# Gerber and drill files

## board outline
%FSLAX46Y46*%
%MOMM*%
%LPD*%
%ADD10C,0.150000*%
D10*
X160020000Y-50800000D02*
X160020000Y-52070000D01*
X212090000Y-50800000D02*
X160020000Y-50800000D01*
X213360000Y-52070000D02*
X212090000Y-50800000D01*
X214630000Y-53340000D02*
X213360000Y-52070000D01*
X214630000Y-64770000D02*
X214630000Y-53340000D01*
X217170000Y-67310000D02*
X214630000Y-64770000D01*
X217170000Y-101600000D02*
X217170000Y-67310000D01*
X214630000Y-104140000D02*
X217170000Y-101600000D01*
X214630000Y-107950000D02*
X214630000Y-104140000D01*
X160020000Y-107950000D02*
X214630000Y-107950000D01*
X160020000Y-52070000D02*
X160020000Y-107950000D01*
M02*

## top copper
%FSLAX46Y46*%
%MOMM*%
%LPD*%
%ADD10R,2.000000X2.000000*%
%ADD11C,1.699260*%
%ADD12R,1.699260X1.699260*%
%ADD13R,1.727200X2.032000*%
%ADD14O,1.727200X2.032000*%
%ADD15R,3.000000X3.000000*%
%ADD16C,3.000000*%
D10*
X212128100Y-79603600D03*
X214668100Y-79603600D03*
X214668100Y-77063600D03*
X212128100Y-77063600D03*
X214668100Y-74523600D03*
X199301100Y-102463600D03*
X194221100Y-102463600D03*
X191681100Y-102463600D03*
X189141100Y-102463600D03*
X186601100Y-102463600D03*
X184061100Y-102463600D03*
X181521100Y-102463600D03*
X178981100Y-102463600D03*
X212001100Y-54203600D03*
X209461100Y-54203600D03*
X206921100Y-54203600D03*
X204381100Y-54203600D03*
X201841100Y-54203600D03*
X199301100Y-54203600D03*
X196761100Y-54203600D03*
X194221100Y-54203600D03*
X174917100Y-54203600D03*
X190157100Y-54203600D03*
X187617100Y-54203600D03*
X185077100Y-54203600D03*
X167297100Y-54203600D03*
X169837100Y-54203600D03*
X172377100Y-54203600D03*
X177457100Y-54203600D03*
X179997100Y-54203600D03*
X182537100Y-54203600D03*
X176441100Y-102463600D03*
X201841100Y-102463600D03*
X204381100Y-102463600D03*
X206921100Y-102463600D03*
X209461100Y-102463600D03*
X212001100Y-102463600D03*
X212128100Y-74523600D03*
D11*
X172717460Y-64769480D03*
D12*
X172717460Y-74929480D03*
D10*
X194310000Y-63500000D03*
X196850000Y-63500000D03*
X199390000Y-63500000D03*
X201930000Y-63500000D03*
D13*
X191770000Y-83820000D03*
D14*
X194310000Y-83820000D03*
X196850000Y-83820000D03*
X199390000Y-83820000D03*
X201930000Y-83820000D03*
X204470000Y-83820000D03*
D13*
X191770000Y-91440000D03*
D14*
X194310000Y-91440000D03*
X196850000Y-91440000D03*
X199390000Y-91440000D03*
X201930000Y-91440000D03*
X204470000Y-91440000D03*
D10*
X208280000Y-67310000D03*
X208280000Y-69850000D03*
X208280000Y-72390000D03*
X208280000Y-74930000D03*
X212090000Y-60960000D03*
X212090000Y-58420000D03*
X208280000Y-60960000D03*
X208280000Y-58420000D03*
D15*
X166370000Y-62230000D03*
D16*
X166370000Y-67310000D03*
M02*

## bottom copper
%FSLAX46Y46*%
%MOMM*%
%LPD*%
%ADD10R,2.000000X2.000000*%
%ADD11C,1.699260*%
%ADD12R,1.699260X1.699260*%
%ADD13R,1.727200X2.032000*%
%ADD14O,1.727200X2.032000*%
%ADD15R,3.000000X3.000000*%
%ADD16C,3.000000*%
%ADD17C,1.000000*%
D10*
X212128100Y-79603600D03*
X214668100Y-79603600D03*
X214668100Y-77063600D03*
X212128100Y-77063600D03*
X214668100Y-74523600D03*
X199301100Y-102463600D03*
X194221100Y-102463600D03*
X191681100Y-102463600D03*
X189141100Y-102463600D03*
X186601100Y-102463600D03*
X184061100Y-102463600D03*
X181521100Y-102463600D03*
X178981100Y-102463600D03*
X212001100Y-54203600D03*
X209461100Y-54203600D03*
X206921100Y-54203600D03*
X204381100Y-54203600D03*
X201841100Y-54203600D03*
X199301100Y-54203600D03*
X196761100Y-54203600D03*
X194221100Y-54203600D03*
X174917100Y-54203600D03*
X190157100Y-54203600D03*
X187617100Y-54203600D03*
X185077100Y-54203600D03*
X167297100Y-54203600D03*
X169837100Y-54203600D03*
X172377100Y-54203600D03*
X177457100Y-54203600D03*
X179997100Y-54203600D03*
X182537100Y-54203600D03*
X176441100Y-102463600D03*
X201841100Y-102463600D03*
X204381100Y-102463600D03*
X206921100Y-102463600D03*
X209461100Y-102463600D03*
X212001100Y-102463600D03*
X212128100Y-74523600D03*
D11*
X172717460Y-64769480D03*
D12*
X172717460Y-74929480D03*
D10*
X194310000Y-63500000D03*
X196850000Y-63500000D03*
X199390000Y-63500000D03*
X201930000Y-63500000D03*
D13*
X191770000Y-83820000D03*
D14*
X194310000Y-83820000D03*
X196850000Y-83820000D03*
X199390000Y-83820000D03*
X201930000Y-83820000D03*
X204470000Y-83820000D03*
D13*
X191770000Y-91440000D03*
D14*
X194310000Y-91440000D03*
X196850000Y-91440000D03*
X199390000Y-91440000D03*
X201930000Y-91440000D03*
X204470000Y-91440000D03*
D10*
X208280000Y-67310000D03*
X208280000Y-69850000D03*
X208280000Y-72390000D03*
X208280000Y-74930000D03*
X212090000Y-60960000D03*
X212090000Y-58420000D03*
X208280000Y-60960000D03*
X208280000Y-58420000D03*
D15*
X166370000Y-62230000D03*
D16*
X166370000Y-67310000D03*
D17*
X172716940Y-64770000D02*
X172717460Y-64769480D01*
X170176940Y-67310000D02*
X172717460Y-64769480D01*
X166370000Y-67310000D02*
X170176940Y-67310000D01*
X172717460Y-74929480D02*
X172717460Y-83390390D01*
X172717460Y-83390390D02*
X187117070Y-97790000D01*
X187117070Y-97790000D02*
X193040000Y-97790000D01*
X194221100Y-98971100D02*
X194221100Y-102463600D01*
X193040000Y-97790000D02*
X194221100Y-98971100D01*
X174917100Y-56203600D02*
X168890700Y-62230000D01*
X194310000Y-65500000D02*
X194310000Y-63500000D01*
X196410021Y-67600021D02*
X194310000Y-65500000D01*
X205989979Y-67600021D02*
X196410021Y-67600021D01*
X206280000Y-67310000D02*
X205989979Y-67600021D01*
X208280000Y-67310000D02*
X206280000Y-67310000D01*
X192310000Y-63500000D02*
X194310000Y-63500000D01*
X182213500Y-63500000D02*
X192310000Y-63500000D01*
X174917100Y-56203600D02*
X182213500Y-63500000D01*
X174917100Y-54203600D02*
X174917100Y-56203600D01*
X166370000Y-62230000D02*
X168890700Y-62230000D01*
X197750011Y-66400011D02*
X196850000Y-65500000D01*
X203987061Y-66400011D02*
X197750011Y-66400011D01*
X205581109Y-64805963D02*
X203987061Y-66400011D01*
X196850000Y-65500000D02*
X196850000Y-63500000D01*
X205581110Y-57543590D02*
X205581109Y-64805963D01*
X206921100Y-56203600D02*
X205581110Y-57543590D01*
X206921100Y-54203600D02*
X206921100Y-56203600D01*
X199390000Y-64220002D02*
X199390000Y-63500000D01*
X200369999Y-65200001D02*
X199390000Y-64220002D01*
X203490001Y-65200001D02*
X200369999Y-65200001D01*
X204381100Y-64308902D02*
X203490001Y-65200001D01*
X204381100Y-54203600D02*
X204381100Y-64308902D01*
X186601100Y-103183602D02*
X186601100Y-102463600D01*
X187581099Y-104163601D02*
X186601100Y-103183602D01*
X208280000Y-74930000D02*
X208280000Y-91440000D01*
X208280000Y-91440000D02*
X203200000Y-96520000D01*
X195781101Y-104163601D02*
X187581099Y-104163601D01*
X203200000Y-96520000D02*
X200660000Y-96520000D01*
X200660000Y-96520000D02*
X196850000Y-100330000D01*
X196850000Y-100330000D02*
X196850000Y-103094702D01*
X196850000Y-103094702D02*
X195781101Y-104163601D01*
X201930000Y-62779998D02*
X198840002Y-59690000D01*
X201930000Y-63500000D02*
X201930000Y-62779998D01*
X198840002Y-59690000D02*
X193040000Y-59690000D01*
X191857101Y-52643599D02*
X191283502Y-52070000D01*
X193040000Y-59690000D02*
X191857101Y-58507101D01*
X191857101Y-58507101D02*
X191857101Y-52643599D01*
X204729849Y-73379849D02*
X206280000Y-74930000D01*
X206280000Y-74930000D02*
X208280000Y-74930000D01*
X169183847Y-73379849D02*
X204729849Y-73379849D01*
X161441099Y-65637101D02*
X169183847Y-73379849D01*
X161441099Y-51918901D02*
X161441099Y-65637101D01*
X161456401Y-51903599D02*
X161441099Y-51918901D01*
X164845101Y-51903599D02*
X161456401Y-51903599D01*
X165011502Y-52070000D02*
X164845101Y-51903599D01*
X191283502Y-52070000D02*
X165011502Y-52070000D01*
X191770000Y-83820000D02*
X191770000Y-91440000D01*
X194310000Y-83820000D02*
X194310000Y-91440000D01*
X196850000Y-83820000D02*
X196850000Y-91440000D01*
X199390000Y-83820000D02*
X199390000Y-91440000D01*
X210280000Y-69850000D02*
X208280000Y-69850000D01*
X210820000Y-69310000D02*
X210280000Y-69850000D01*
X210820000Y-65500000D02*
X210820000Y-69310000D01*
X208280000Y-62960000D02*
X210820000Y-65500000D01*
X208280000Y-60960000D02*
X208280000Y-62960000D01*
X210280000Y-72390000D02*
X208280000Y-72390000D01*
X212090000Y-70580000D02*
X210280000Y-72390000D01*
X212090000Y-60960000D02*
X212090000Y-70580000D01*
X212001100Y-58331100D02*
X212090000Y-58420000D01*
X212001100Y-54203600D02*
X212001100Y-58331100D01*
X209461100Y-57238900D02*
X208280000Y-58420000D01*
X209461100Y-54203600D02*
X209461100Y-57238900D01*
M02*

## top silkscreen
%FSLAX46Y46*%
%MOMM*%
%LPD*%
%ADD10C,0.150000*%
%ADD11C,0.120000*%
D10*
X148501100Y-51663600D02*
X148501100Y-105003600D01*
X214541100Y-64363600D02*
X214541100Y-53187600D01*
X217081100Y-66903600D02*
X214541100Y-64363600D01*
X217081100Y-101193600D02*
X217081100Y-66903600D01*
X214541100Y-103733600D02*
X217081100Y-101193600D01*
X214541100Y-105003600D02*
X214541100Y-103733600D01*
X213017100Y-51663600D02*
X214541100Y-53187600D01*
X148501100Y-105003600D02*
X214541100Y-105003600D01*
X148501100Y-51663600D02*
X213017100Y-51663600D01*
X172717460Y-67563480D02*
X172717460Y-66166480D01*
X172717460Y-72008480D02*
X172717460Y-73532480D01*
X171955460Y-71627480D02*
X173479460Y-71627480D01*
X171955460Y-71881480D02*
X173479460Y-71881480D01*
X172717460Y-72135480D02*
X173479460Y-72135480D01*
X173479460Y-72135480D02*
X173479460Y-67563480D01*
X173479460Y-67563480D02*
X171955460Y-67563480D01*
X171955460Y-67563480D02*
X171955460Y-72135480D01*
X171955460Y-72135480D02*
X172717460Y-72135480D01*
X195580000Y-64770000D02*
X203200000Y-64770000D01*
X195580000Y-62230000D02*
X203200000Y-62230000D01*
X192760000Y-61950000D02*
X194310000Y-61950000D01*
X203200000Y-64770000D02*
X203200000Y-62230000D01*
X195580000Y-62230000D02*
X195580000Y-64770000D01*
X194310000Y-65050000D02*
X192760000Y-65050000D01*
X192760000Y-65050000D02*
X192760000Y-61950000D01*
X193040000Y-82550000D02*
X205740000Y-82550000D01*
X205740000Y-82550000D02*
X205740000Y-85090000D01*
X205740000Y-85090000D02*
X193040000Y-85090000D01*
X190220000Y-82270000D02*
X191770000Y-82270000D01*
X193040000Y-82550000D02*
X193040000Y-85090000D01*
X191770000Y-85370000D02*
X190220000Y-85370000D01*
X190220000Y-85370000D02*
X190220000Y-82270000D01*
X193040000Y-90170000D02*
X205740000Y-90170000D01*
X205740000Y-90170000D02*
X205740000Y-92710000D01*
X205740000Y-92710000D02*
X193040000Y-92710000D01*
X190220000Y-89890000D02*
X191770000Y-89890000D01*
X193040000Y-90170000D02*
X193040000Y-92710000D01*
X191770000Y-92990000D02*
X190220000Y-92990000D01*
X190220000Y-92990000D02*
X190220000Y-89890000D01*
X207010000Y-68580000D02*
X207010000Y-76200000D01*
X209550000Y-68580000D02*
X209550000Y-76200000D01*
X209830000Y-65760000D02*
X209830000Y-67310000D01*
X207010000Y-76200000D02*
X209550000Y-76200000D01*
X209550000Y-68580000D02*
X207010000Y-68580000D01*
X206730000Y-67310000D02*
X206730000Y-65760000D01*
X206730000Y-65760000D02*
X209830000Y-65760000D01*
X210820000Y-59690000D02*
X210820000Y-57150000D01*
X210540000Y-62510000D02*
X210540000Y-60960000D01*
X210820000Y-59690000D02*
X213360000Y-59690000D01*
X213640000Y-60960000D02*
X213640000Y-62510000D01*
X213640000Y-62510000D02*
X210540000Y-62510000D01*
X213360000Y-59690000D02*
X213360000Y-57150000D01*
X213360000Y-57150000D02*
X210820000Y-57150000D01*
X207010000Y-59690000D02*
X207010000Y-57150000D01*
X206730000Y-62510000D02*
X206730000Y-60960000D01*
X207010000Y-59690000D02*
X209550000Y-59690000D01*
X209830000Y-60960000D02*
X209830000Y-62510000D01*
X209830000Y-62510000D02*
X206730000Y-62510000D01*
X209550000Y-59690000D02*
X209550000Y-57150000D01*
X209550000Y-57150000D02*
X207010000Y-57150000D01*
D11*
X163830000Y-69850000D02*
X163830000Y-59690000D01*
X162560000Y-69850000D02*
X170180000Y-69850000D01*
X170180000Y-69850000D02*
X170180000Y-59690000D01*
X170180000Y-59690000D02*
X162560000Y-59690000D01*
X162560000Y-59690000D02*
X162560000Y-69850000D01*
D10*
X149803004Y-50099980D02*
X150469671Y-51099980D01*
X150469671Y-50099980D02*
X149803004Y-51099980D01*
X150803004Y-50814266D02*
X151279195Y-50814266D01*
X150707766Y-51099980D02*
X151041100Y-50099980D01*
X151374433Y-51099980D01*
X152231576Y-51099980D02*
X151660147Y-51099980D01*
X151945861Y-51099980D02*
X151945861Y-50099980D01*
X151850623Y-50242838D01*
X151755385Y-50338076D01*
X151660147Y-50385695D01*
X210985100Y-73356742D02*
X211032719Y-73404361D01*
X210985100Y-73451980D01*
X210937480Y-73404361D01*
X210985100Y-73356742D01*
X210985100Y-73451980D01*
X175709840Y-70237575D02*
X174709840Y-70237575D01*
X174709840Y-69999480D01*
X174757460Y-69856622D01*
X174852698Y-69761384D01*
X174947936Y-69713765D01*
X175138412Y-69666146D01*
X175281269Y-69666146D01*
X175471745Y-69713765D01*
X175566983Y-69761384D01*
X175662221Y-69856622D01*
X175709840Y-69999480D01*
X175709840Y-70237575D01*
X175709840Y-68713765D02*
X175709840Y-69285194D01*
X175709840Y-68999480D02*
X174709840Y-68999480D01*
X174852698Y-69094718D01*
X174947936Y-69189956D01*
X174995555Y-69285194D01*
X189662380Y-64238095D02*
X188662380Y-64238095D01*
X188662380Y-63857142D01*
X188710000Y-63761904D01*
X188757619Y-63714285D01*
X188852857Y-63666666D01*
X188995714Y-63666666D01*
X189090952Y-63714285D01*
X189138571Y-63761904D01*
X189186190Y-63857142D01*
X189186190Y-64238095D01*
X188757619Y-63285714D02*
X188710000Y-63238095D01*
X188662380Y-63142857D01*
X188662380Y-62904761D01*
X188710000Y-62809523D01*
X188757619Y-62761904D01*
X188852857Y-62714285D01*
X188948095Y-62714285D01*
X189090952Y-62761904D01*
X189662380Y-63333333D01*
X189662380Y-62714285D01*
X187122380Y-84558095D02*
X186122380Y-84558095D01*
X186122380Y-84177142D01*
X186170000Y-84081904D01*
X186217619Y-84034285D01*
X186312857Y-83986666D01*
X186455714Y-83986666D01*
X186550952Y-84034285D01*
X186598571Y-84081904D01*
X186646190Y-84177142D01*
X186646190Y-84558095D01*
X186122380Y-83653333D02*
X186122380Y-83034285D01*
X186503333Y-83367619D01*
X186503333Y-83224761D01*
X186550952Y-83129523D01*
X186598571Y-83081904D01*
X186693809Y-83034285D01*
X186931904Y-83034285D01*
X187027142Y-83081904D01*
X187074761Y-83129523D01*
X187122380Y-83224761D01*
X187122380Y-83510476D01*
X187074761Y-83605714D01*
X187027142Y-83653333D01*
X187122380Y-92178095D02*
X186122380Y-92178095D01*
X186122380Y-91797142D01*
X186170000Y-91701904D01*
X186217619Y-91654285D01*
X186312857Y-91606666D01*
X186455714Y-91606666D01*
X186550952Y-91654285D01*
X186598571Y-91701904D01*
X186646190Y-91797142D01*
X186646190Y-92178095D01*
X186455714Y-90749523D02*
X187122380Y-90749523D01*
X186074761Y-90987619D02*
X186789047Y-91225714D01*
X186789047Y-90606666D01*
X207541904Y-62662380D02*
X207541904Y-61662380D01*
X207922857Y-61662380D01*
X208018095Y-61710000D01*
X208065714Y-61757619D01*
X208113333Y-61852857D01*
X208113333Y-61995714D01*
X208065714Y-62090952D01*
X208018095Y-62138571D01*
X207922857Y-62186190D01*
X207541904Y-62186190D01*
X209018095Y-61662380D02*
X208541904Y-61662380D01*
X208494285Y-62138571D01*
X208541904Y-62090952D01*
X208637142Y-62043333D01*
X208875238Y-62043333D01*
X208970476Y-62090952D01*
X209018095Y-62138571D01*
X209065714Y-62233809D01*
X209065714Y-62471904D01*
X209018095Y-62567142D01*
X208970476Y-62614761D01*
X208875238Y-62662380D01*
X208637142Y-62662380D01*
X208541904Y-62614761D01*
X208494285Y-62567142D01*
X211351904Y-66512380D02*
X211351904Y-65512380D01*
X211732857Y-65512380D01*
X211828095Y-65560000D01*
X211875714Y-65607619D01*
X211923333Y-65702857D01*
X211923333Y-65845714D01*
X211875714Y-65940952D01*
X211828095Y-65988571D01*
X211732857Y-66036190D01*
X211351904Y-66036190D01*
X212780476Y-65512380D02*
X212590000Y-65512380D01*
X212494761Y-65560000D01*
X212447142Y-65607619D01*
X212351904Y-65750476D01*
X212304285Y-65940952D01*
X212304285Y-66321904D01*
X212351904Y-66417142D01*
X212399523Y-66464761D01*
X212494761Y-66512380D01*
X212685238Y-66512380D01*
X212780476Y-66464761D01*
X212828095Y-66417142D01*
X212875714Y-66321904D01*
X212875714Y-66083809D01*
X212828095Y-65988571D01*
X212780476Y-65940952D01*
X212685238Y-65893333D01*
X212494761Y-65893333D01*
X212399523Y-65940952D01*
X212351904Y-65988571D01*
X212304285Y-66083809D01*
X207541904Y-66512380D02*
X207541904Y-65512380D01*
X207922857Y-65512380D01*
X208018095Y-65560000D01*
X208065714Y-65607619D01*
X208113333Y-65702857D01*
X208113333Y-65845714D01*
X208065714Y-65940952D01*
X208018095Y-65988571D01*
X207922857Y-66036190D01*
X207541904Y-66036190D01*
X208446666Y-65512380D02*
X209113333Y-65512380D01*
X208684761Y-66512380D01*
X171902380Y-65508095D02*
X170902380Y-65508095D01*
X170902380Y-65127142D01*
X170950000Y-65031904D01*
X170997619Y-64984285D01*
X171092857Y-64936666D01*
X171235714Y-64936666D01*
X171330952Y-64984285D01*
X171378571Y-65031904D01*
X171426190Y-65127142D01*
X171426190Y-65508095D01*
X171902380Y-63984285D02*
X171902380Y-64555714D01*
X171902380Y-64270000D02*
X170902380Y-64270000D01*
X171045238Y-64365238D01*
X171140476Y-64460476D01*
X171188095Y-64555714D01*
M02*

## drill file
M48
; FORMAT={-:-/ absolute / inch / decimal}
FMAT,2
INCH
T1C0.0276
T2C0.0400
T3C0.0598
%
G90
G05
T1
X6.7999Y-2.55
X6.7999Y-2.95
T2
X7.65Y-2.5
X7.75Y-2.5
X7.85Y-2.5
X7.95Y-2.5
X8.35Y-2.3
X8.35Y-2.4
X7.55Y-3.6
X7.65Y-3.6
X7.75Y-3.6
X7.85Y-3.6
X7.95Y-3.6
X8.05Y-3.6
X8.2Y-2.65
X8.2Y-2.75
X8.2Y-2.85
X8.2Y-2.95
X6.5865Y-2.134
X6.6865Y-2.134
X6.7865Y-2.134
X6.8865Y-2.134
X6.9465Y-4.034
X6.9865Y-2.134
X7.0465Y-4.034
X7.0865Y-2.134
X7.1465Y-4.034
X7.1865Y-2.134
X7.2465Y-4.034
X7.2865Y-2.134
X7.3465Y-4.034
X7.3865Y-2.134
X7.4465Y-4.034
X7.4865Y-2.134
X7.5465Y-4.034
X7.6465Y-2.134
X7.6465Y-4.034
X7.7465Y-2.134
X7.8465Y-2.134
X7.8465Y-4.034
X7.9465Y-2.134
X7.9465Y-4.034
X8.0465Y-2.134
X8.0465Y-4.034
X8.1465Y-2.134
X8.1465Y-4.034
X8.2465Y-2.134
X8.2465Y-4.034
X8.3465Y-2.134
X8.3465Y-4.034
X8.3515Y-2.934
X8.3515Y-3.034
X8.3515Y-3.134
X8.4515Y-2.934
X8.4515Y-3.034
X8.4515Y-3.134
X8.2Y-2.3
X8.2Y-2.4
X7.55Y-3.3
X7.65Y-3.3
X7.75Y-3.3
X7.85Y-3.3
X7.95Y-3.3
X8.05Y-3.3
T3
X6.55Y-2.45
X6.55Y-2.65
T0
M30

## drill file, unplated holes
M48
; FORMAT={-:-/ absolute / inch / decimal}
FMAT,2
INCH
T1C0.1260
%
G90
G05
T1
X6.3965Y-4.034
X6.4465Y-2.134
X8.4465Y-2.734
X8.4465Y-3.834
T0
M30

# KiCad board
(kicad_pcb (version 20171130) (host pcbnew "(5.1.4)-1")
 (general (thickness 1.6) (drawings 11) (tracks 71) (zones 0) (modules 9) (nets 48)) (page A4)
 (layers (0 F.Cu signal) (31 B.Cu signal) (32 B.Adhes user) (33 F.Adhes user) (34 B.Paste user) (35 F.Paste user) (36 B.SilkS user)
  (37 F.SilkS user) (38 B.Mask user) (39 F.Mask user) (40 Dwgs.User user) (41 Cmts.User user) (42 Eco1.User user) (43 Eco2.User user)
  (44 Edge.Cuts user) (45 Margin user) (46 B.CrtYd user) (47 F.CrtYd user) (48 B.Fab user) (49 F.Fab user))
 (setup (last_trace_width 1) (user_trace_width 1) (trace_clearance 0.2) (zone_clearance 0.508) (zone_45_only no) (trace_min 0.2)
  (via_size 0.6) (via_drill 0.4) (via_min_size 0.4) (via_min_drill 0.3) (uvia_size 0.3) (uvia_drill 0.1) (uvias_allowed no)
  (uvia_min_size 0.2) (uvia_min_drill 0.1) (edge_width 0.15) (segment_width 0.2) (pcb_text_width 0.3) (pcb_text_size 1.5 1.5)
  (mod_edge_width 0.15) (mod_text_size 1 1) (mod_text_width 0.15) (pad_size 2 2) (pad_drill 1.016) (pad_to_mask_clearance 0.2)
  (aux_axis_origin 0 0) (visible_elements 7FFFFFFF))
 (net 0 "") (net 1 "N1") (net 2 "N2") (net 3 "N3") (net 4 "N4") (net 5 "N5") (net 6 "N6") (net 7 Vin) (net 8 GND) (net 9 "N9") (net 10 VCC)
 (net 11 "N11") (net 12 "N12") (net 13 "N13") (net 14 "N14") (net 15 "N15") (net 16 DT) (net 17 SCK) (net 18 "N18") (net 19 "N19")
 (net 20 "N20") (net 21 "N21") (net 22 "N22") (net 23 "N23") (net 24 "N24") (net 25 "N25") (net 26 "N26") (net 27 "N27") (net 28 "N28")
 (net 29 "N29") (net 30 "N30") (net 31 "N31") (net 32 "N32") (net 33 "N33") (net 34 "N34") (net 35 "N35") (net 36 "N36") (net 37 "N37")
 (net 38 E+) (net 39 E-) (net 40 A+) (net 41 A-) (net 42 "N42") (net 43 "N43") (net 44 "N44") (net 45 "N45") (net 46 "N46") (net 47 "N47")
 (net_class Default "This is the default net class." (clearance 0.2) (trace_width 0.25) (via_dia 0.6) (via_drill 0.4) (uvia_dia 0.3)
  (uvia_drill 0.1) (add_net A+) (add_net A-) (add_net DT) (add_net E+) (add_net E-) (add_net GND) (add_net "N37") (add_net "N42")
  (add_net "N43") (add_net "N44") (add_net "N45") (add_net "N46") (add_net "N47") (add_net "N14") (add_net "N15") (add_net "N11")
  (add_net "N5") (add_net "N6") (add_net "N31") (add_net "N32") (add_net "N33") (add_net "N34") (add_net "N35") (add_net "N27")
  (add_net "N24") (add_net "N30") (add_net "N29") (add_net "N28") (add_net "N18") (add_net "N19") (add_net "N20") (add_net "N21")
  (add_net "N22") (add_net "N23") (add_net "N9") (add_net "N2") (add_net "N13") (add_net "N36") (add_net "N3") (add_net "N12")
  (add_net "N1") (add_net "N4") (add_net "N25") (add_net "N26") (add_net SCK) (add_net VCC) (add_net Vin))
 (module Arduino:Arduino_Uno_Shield (layer F.Cu) (at 148.5011 105.0036)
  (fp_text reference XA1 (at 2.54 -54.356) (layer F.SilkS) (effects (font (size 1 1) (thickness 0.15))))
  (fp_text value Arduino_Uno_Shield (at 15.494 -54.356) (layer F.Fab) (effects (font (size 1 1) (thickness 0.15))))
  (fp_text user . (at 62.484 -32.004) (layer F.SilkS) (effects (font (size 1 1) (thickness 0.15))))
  (fp_line (start 0 -53.34) (end 0 0) (layer F.SilkS) (width 0.15))
  (fp_line (start 66.04 -40.64) (end 66.04 -51.816) (layer F.SilkS) (width 0.15))
  (fp_line (start 68.58 -38.1) (end 66.04 -40.64) (layer F.SilkS) (width 0.15))
  (fp_line (start 68.58 -3.81) (end 68.58 -38.1) (layer F.SilkS) (width 0.15))
  (fp_line (start 66.04 -1.27) (end 68.58 -3.81) (layer F.SilkS) (width 0.15))
  (fp_line (start 66.04 0) (end 66.04 -1.27) (layer F.SilkS) (width 0.15))
  (fp_line (start 64.516 -53.34) (end 66.04 -51.816) (layer F.SilkS) (width 0.15))
  (fp_line (start 0 0) (end 66.04 0) (layer F.SilkS) (width 0.15))
  (fp_line (start 0 -53.34) (end 64.516 -53.34) (layer F.SilkS) (width 0.15))
  (pad RST2 thru_hole rect (at 63.627 -25.4) (size 2 2) (drill 1.016) (layers *.Cu *.Mask) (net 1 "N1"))
  (pad GND4 thru_hole rect (at 66.167 -25.4) (size 2 2) (drill 1.016) (layers *.Cu *.Mask) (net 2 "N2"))
  (pad MOSI thru_hole rect (at 66.167 -27.94) (size 2 2) (drill 1.016) (layers *.Cu *.Mask) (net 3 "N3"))
  (pad SCK thru_hole rect (at 63.627 -27.94) (size 2 2) (drill 1.016) (layers *.Cu *.Mask) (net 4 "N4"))
  (pad 5V2 thru_hole rect (at 66.167 -30.48) (size 2 2) (drill 1.016) (layers *.Cu *.Mask) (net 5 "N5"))
  (pad A0 thru_hole rect (at 50.8 -2.54) (size 2 2) (drill 1.016) (layers *.Cu *.Mask) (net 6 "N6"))
  (pad VIN thru_hole rect (at 45.72 -2.54) (size 2 2) (drill 1.016) (layers *.Cu *.Mask) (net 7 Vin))
  (pad GND3 thru_hole rect (at 43.18 -2.54) (size 2 2) (drill 1.016) (layers *.Cu *.Mask) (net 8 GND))
  (pad GND2 thru_hole rect (at 40.64 -2.54) (size 2 2) (drill 1.016) (layers *.Cu *.Mask) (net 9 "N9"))
  (pad 5V1 thru_hole rect (at 38.1 -2.54) (size 2 2) (drill 1.016) (layers *.Cu *.Mask) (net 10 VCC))
  (pad 3V3 thru_hole rect (at 35.56 -2.54) (size 2 2) (drill 1.016) (layers *.Cu *.Mask) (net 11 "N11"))
  (pad RST1 thru_hole rect (at 33.02 -2.54) (size 2 2) (drill 1.016) (layers *.Cu *.Mask) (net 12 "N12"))
  (pad IORF thru_hole rect (at 30.48 -2.54) (size 2 2) (drill 1.016) (layers *.Cu *.Mask) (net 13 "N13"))
  (pad D0 thru_hole rect (at 63.5 -50.8) (size 2 2) (drill 1.016) (layers *.Cu *.Mask) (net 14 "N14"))
  (pad D1 thru_hole rect (at 60.96 -50.8) (size 2 2) (drill 1.016) (layers *.Cu *.Mask) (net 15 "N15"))
  (pad D2 thru_hole rect (at 58.42 -50.8) (size 2 2) (drill 1.016) (layers *.Cu *.Mask) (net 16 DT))
  (pad D3 thru_hole rect (at 55.88 -50.8) (size 2 2) (drill 1.016) (layers *.Cu *.Mask) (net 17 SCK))
  (pad D4 thru_hole rect (at 53.34 -50.8) (size 2 2) (drill 1.016) (layers *.Cu *.Mask) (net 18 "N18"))
  (pad D5 thru_hole rect (at 50.8 -50.8) (size 2 2) (drill 1.016) (layers *.Cu *.Mask) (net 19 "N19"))
  (pad D6 thru_hole rect (at 48.26 -50.8) (size 2 2) (drill 1.016) (layers *.Cu *.Mask) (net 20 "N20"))
  (pad D7 thru_hole rect (at 45.72 -50.8) (size 2 2) (drill 1.016) (layers *.Cu *.Mask) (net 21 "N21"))
  (pad GND1 thru_hole rect (at 26.416 -50.8) (size 2 2) (drill 1.016) (layers *.Cu *.Mask) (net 8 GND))
  (pad D8 thru_hole rect (at 41.656 -50.8) (size 2 2) (drill 1.016) (layers *.Cu *.Mask) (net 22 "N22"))
  (pad D9 thru_hole rect (at 39.116 -50.8) (size 2 2) (drill 1.016) (layers *.Cu *.Mask) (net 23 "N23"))
  (pad D10 thru_hole rect (at 36.576 -50.8) (size 2 2) (drill 1.016) (layers *.Cu *.Mask) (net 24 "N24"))
  (pad "" np_thru_hole circle (at 66.04 -7.62) (size 3.2 3.2) (drill 3.2) (layers *.Cu *.Mask))
  (pad "" np_thru_hole circle (at 66.04 -35.56) (size 3.2 3.2) (drill 3.2) (layers *.Cu *.Mask))
  (pad "" np_thru_hole circle (at 15.24 -50.8) (size 3.2 3.2) (drill 3.2) (layers *.Cu *.Mask))
  (pad "" np_thru_hole circle (at 13.97 -2.54) (size 3.2 3.2) (drill 3.2) (layers *.Cu *.Mask))
  (pad SCL thru_hole rect (at 18.796 -50.8) (size 2 2) (drill 1.016) (layers *.Cu *.Mask) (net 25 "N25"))
  (pad SDA thru_hole rect (at 21.336 -50.8) (size 2 2) (drill 1.016) (layers *.Cu *.Mask) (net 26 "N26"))
  (pad AREF thru_hole rect (at 23.876 -50.8) (size 2 2) (drill 1.016) (layers *.Cu *.Mask) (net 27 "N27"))
  (pad D13 thru_hole rect (at 28.956 -50.8) (size 2 2) (drill 1.016) (layers *.Cu *.Mask) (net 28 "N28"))
  (pad D12 thru_hole rect (at 31.496 -50.8) (size 2 2) (drill 1.016) (layers *.Cu *.Mask) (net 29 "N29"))
  (pad D11 thru_hole rect (at 34.036 -50.8) (size 2 2) (drill 1.016) (layers *.Cu *.Mask) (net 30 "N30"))
  (pad "" thru_hole rect (at 27.94 -2.54) (size 2 2) (drill 1.016) (layers *.Cu *.Mask))
  (pad A1 thru_hole rect (at 53.34 -2.54) (size 2 2) (drill 1.016) (layers *.Cu *.Mask) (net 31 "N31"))
  (pad A2 thru_hole rect (at 55.88 -2.54) (size 2 2) (drill 1.016) (layers *.Cu *.Mask) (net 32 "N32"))
  (pad A3 thru_hole rect (at 58.42 -2.54) (size 2 2) (drill 1.016) (layers *.Cu *.Mask) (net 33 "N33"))
  (pad A4 thru_hole rect (at 60.96 -2.54) (size 2 2) (drill 1.016) (layers *.Cu *.Mask) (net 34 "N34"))
  (pad A5 thru_hole rect (at 63.5 -2.54) (size 2 2) (drill 1.016) (layers *.Cu *.Mask) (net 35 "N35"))
  (pad MISO thru_hole rect (at 63.627 -30.48) (size 2 2) (drill 1.016) (layers *.Cu *.Mask) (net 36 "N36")))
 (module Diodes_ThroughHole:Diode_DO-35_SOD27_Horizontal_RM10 (layer F.Cu) (at 172.72 74.93 90)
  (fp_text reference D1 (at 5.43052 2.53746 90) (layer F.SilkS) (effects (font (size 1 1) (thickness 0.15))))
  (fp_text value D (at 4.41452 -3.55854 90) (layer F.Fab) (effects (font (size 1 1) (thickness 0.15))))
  (fp_line (start 7.36652 -0.00254) (end 8.76352 -0.00254) (layer F.SilkS) (width 0.15))
  (fp_line (start 2.92152 -0.00254) (end 1.39752 -0.00254) (layer F.SilkS) (width 0.15))
  (fp_line (start 3.30252 -0.76454) (end 3.30252 0.75946) (layer F.SilkS) (width 0.15))
  (fp_line (start 3.04852 -0.76454) (end 3.04852 0.75946) (layer F.SilkS) (width 0.15))
  (fp_line (start 2.79452 -0.00254) (end 2.79452 0.75946) (layer F.SilkS) (width 0.15))
  (fp_line (start 2.79452 0.75946) (end 7.36652 0.75946) (layer F.SilkS) (width 0.15))
  (fp_line (start 7.36652 0.75946) (end 7.36652 -0.76454) (layer F.SilkS) (width 0.15))
  (fp_line (start 7.36652 -0.76454) (end 2.79452 -0.76454) (layer F.SilkS) (width 0.15))
  (fp_line (start 2.79452 -0.76454) (end 2.79452 -0.00254) (layer F.SilkS) (width 0.15))
  (pad 2 thru_hole circle (at 10.16052 -0.00254 270) (size 1.69926 1.69926) (drill 0.70104) (layers *.Cu *.Mask F.SilkS) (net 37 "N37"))
  (pad 1 thru_hole rect (at 0.00052 -0.00254 270) (size 1.69926 1.69926) (drill 0.70104) (layers *.Cu *.Mask F.SilkS) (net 7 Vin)))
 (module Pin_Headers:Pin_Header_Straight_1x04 (layer F.Cu) (at 194.31 63.5 90)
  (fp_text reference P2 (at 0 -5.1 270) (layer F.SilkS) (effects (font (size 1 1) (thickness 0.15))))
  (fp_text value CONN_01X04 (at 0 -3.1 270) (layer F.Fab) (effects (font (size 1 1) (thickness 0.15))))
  (fp_line (start -1.27 1.27) (end -1.27 8.89) (layer F.SilkS) (width 0.15))
  (fp_line (start 1.27 1.27) (end 1.27 8.89) (layer F.SilkS) (width 0.15))
  (fp_line (start 1.55 -1.55) (end 1.55 0) (layer F.SilkS) (width 0.15))
  (fp_line (start -1.27 8.89) (end 1.27 8.89) (layer F.SilkS) (width 0.15))
  (fp_line (start 1.27 1.27) (end -1.27 1.27) (layer F.SilkS) (width 0.15))
  (fp_line (start -1.55 0) (end -1.55 -1.55) (layer F.SilkS) (width 0.15))
  (fp_line (start -1.55 -1.55) (end 1.55 -1.55) (layer F.SilkS) (width 0.15))
  (pad 1 thru_hole rect (at 0 0 90) (size 2 2) (drill 1.016) (layers *.Cu *.Mask) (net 8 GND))
  (pad 2 thru_hole rect (at 0 2.54 90) (size 2 2) (drill 1.016) (layers *.Cu *.Mask) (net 16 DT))
  (pad 3 thru_hole rect (at 0 5.08 90) (size 2 2) (drill 1.016) (layers *.Cu *.Mask) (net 17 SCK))
  (pad 4 thru_hole rect (at 0 7.62 90) (size 2 2) (drill 1.016) (layers *.Cu *.Mask) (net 10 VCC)))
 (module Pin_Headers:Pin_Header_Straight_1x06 (layer F.Cu) (at 191.77 83.82 90)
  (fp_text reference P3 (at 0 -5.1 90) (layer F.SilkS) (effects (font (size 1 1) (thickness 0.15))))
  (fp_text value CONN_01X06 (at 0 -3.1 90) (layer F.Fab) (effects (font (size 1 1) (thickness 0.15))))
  (fp_line (start 1.27 1.27) (end 1.27 13.97) (layer F.SilkS) (width 0.15))
  (fp_line (start 1.27 13.97) (end -1.27 13.97) (layer F.SilkS) (width 0.15))
  (fp_line (start -1.27 13.97) (end -1.27 1.27) (layer F.SilkS) (width 0.15))
  (fp_line (start 1.55 -1.55) (end 1.55 0) (layer F.SilkS) (width 0.15))
  (fp_line (start 1.27 1.27) (end -1.27 1.27) (layer F.SilkS) (width 0.15))
  (fp_line (start -1.55 0) (end -1.55 -1.55) (layer F.SilkS) (width 0.15))
  (fp_line (start -1.55 -1.55) (end 1.55 -1.55) (layer F.SilkS) (width 0.15))
  (pad 1 thru_hole rect (at 0 0 90) (size 2.032 1.7272) (drill 1.016) (layers *.Cu *.Mask F.SilkS) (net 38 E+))
  (pad 2 thru_hole oval (at 0 2.54 90) (size 2.032 1.7272) (drill 1.016) (layers *.Cu *.Mask F.SilkS) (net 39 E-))
  (pad 3 thru_hole oval (at 0 5.08 90) (size 2.032 1.7272) (drill 1.016) (layers *.Cu *.Mask F.SilkS) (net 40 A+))
  (pad 4 thru_hole oval (at 0 7.62 90) (size 2.032 1.7272) (drill 1.016) (layers *.Cu *.Mask F.SilkS) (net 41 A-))
  (pad 5 thru_hole oval (at 0 10.16 90) (size 2.032 1.7272) (drill 1.016) (layers *.Cu *.Mask F.SilkS) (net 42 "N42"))
  (pad 6 thru_hole oval (at 0 12.7 90) (size 2.032 1.7272) (drill 1.016) (layers *.Cu *.Mask F.SilkS) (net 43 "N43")))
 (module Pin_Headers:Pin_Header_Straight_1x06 (layer F.Cu) (at 191.77 91.44 90)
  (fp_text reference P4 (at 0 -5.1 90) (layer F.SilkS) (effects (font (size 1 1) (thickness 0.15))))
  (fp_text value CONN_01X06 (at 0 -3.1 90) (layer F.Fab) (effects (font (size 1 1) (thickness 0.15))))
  (fp_line (start 1.27 1.27) (end 1.27 13.97) (layer F.SilkS) (width 0.15))
  (fp_line (start 1.27 13.97) (end -1.27 13.97) (layer F.SilkS) (width 0.15))
  (fp_line (start -1.27 13.97) (end -1.27 1.27) (layer F.SilkS) (width 0.15))
  (fp_line (start 1.55 -1.55) (end 1.55 0) (layer F.SilkS) (width 0.15))
  (fp_line (start 1.27 1.27) (end -1.27 1.27) (layer F.SilkS) (width 0.15))
  (fp_line (start -1.55 0) (end -1.55 -1.55) (layer F.SilkS) (width 0.15))
  (fp_line (start -1.55 -1.55) (end 1.55 -1.55) (layer F.SilkS) (width 0.15))
  (pad 1 thru_hole rect (at 0 0 90) (size 2.032 1.7272) (drill 1.016) (layers *.Cu *.Mask F.SilkS) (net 38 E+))
  (pad 2 thru_hole oval (at 0 2.54 90) (size 2.032 1.7272) (drill 1.016) (layers *.Cu *.Mask F.SilkS) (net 39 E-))
  (pad 3 thru_hole oval (at 0 5.08 90) (size 2.032 1.7272) (drill 1.016) (layers *.Cu *.Mask F.SilkS) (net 40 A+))
  (pad 4 thru_hole oval (at 0 7.62 90) (size 2.032 1.7272) (drill 1.016) (layers *.Cu *.Mask F.SilkS) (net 41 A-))
  (pad 5 thru_hole oval (at 0 10.16 90) (size 2.032 1.7272) (drill 1.016) (layers *.Cu *.Mask F.SilkS) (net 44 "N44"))
  (pad 6 thru_hole oval (at 0 12.7 90) (size 2.032 1.7272) (drill 1.016) (layers *.Cu *.Mask F.SilkS) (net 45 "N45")))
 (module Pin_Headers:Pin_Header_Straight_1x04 (layer F.Cu) (at 208.28 67.31)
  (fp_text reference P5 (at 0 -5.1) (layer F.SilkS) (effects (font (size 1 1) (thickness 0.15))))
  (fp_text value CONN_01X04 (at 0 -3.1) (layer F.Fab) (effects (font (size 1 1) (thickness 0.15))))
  (fp_line (start -1.27 1.27) (end -1.27 8.89) (layer F.SilkS) (width 0.15))
  (fp_line (start 1.27 1.27) (end 1.27 8.89) (layer F.SilkS) (width 0.15))
  (fp_line (start 1.55 -1.55) (end 1.55 0) (layer F.SilkS) (width 0.15))
  (fp_line (start -1.27 8.89) (end 1.27 8.89) (layer F.SilkS) (width 0.15))
  (fp_line (start 1.27 1.27) (end -1.27 1.27) (layer F.SilkS) (width 0.15))
  (fp_line (start -1.55 0) (end -1.55 -1.55) (layer F.SilkS) (width 0.15))
  (fp_line (start -1.55 -1.55) (end 1.55 -1.55) (layer F.SilkS) (width 0.15))
  (pad 1 thru_hole rect (at 0 0) (size 2 2) (drill 1.016) (layers *.Cu *.Mask) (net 8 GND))
  (pad 2 thru_hole rect (at 0 2.54) (size 2 2) (drill 1.016) (layers *.Cu *.Mask) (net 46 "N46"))
  (pad 3 thru_hole rect (at 0 5.08) (size 2 2) (drill 1.016) (layers *.Cu *.Mask) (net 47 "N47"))
  (pad 4 thru_hole rect (at 0 7.62) (size 2 2) (drill 1.016) (layers *.Cu *.Mask) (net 10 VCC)))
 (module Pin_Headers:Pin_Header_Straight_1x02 (layer F.Cu) (at 212.09 60.96 180)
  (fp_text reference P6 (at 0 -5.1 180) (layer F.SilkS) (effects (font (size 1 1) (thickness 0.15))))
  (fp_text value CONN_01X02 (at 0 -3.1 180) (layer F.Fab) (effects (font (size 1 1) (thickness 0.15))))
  (fp_line (start 1.27 1.27) (end 1.27 3.81) (layer F.SilkS) (width 0.15))
  (fp_line (start 1.55 -1.55) (end 1.55 0) (layer F.SilkS) (width 0.15))
  (fp_line (start 1.27 1.27) (end -1.27 1.27) (layer F.SilkS) (width 0.15))
  (fp_line (start -1.55 0) (end -1.55 -1.55) (layer F.SilkS) (width 0.15))
  (fp_line (start -1.55 -1.55) (end 1.55 -1.55) (layer F.SilkS) (width 0.15))
  (fp_line (start -1.27 1.27) (end -1.27 3.81) (layer F.SilkS) (width 0.15))
  (fp_line (start -1.27 3.81) (end 1.27 3.81) (layer F.SilkS) (width 0.15))
  (pad 1 thru_hole rect (at 0 0 180) (size 2 2) (drill 1.016) (layers *.Cu *.Mask) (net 47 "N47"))
  (pad 2 thru_hole rect (at 0 2.54 180) (size 2 2) (drill 1.016) (layers *.Cu *.Mask) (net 14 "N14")))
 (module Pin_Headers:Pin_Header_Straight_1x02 (layer F.Cu) (at 208.28 60.96 180)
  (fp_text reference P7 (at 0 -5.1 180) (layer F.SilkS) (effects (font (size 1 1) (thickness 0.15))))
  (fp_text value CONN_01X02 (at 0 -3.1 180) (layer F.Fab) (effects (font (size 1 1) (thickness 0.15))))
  (fp_line (start 1.27 1.27) (end 1.27 3.81) (layer F.SilkS) (width 0.15))
  (fp_line (start 1.55 -1.55) (end 1.55 0) (layer F.SilkS) (width 0.15))
  (fp_line (start 1.27 1.27) (end -1.27 1.27) (layer F.SilkS) (width 0.15))
  (fp_line (start -1.55 0) (end -1.55 -1.55) (layer F.SilkS) (width 0.15))
  (fp_line (start -1.55 -1.55) (end 1.55 -1.55) (layer F.SilkS) (width 0.15))
  (fp_line (start -1.27 1.27) (end -1.27 3.81) (layer F.SilkS) (width 0.15))
  (fp_line (start -1.27 3.81) (end 1.27 3.81) (layer F.SilkS) (width 0.15))
  (pad 1 thru_hole rect (at 0 0 180) (size 2 2) (drill 1.016) (layers *.Cu *.Mask) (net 46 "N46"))
  (pad 2 thru_hole rect (at 0 2.54 180) (size 2 2) (drill 1.016) (layers *.Cu *.Mask) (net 15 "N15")))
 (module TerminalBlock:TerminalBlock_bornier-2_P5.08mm (layer F.Cu) (at 166.37 62.23 270)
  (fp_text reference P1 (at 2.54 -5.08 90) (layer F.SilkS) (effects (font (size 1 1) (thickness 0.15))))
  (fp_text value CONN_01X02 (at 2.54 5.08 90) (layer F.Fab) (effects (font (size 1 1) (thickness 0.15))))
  (fp_line (start 7.62 2.54) (end -2.54 2.54) (layer F.SilkS) (width 0.12))
  (fp_line (start 7.62 3.81) (end 7.62 -3.81) (layer F.SilkS) (width 0.12))
  (fp_line (start 7.62 -3.81) (end -2.54 -3.81) (layer F.SilkS) (width 0.12))
  (fp_line (start -2.54 -3.81) (end -2.54 3.81) (layer F.SilkS) (width 0.12))
  (fp_line (start -2.54 3.81) (end 7.62 3.81) (layer F.SilkS) (width 0.12))
  (pad 1 thru_hole rect (at 0 0 270) (size 3 3) (drill 1.52) (layers *.Cu *.Mask) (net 8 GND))
  (pad 2 thru_hole circle (at 5.08 0 270) (size 3 3) (drill 1.52) (layers *.Cu *.Mask) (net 37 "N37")))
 (gr_line (start 160.02 50.8) (end 160.02 52.07) (layer Edge.Cuts) (width 0.15))
 (gr_line (start 212.09 50.8) (end 160.02 50.8) (layer Edge.Cuts) (width 0.15))
 (gr_line (start 213.36 52.07) (end 212.09 50.8) (layer Edge.Cuts) (width 0.15))
 (gr_line (start 214.63 53.34) (end 213.36 52.07) (layer Edge.Cuts) (width 0.15))
 (gr_line (start 214.63 64.77) (end 214.63 53.34) (layer Edge.Cuts) (width 0.15))
 (gr_line (start 217.17 67.31) (end 214.63 64.77) (layer Edge.Cuts) (width 0.15))
 (gr_line (start 217.17 101.6) (end 217.17 67.31) (layer Edge.Cuts) (width 0.15))
 (gr_line (start 214.63 104.14) (end 217.17 101.6) (layer Edge.Cuts) (width 0.15))
 (gr_line (start 214.63 107.95) (end 214.63 104.14) (layer Edge.Cuts) (width 0.15))
 (gr_line (start 160.02 107.95) (end 214.63 107.95) (layer Edge.Cuts) (width 0.15))
 (gr_line (start 160.02 52.07) (end 160.02 107.95) (layer Edge.Cuts) (width 0.15))
 (segment (start 172.71694 64.77) (end 172.71746 64.76948) (width 1) (layer B.Cu) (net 37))
 (segment (start 170.17694 67.31) (end 172.71746 64.76948) (width 1) (layer B.Cu) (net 37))
 (segment (start 166.37 67.31) (end 170.17694 67.31) (width 1) (layer B.Cu) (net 37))
 (segment (start 172.71746 74.92948) (end 172.71746 83.39039) (width 1) (layer B.Cu) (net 7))
 (segment (start 172.71746 83.39039) (end 187.11707 97.79) (width 1) (layer B.Cu) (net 7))
 (segment (start 187.11707 97.79) (end 193.04 97.79) (width 1) (layer B.Cu) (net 7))
 (segment (start 194.2211 98.9711) (end 194.2211 102.4636) (width 1) (layer B.Cu) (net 7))
 (segment (start 193.04 97.79) (end 194.2211 98.9711) (width 1) (layer B.Cu) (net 7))
 (segment (start 174.9171 56.2036) (end 168.8907 62.23) (width 1) (layer B.Cu) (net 8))
 (segment (start 194.31 65.5) (end 194.31 63.5) (width 1) (layer B.Cu) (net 8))
 (segment (start 196.410021 67.600021) (end 194.31 65.5) (width 1) (layer B.Cu) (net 8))
 (segment (start 205.989979 67.600021) (end 196.410021 67.600021) (width 1) (layer B.Cu) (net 8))
 (segment (start 206.28 67.31) (end 205.989979 67.600021) (width 1) (layer B.Cu) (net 8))
 (segment (start 208.28 67.31) (end 206.28 67.31) (width 1) (layer B.Cu) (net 8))
 (segment (start 192.31 63.5) (end 194.31 63.5) (width 1) (layer B.Cu) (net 8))
 (segment (start 182.2135 63.5) (end 192.31 63.5) (width 1) (layer B.Cu) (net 8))
 (segment (start 174.9171 56.2036) (end 182.2135 63.5) (width 1) (layer B.Cu) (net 8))
 (segment (start 174.9171 54.2036) (end 174.9171 56.2036) (width 1) (layer B.Cu) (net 8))
 (segment (start 166.37 62.23) (end 168.8907 62.23) (width 1) (layer B.Cu) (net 8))
 (segment (start 197.750011 66.400011) (end 196.85 65.5) (width 1) (layer B.Cu) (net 16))
 (segment (start 203.987061 66.400011) (end 197.750011 66.400011) (width 1) (layer B.Cu) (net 16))
 (segment (start 205.581109 64.805963) (end 203.987061 66.400011) (width 1) (layer B.Cu) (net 16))
 (segment (start 196.85 65.5) (end 196.85 63.5) (width 1) (layer B.Cu) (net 16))
 (segment (start 205.58111 57.54359) (end 205.581109 64.805963) (width 1) (layer B.Cu) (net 16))
 (segment (start 206.9211 56.2036) (end 205.58111 57.54359) (width 1) (layer B.Cu) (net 16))
 (segment (start 206.9211 54.2036) (end 206.9211 56.2036) (width 1) (layer B.Cu) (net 16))
 (segment (start 199.39 64.220002) (end 199.39 63.5) (width 1) (layer B.Cu) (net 17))
 (segment (start 200.369999 65.200001) (end 199.39 64.220002) (width 1) (layer B.Cu) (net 17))
 (segment (start 203.490001 65.200001) (end 200.369999 65.200001) (width 1) (layer B.Cu) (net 17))
 (segment (start 204.3811 64.308902) (end 203.490001 65.200001) (width 1) (layer B.Cu) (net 17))
 (segment (start 204.3811 54.2036) (end 204.3811 64.308902) (width 1) (layer B.Cu) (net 17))
 (segment (start 186.6011 103.183602) (end 186.6011 102.4636) (width 1) (layer B.Cu) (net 10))
 (segment (start 187.581099 104.163601) (end 186.6011 103.183602) (width 1) (layer B.Cu) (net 10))
 (segment (start 208.28 74.93) (end 208.28 91.44) (width 1) (layer B.Cu) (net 10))
 (segment (start 208.28 91.44) (end 203.2 96.52) (width 1) (layer B.Cu) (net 10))
 (segment (start 195.781101 104.163601) (end 187.581099 104.163601) (width 1) (layer B.Cu) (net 10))
 (segment (start 203.2 96.52) (end 200.66 96.52) (width 1) (layer B.Cu) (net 10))
 (segment (start 200.66 96.52) (end 196.85 100.33) (width 1) (layer B.Cu) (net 10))
 (segment (start 196.85 100.33) (end 196.85 103.094702) (width 1) (layer B.Cu) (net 10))
 (segment (start 196.85 103.094702) (end 195.781101 104.163601) (width 1) (layer B.Cu) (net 10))
 (segment (start 201.93 62.779998) (end 198.840002 59.69) (width 1) (layer B.Cu) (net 10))
 (segment (start 201.93 63.5) (end 201.93 62.779998) (width 1) (layer B.Cu) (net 10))
 (segment (start 198.840002 59.69) (end 193.04 59.69) (width 1) (layer B.Cu) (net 10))
 (segment (start 191.857101 52.643599) (end 191.283502 52.07) (width 1) (layer B.Cu) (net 10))
 (segment (start 193.04 59.69) (end 191.857101 58.507101) (width 1) (layer B.Cu) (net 10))
 (segment (start 191.857101 58.507101) (end 191.857101 52.643599) (width 1) (layer B.Cu) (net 10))
 (segment (start 204.729849 73.379849) (end 206.28 74.93) (width 1) (layer B.Cu) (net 10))
 (segment (start 206.28 74.93) (end 208.28 74.93) (width 1) (layer B.Cu) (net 10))
 (segment (start 169.183847 73.379849) (end 204.729849 73.379849) (width 1) (layer B.Cu) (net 10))
 (segment (start 161.441099 65.637101) (end 169.183847 73.379849) (width 1) (layer B.Cu) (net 10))
 (segment (start 161.441099 51.918901) (end 161.441099 65.637101) (width 1) (layer B.Cu) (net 10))
 (segment (start 161.456401 51.903599) (end 161.441099 51.918901) (width 1) (layer B.Cu) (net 10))
 (segment (start 164.845101 51.903599) (end 161.456401 51.903599) (width 1) (layer B.Cu) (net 10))
 (segment (start 165.011502 52.07) (end 164.845101 51.903599) (width 1) (layer B.Cu) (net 10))
 (segment (start 191.283502 52.07) (end 165.011502 52.07) (width 1) (layer B.Cu) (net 10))
 (segment (start 191.77 83.82) (end 191.77 91.44) (width 1) (layer B.Cu) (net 38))
 (segment (start 194.31 83.82) (end 194.31 91.44) (width 1) (layer B.Cu) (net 39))
 (segment (start 196.85 83.82) (end 196.85 91.44) (width 1) (layer B.Cu) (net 40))
 (segment (start 199.39 83.82) (end 199.39 91.44) (width 1) (layer B.Cu) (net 41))
 (segment (start 210.28 69.85) (end 208.28 69.85) (width 1) (layer B.Cu) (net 46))
 (segment (start 210.82 69.31) (end 210.28 69.85) (width 1) (layer B.Cu) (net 46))
 (segment (start 210.82 65.5) (end 210.82 69.31) (width 1) (layer B.Cu) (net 46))
 (segment (start 208.28 62.96) (end 210.82 65.5) (width 1) (layer B.Cu) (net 46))
 (segment (start 208.28 60.96) (end 208.28 62.96) (width 1) (layer B.Cu) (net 46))
 (segment (start 210.28 72.39) (end 208.28 72.39) (width 1) (layer B.Cu) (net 47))
 (segment (start 212.09 70.58) (end 210.28 72.39) (width 1) (layer B.Cu) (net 47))
 (segment (start 212.09 60.96) (end 212.09 70.58) (width 1) (layer B.Cu) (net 47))
 (segment (start 212.0011 58.3311) (end 212.09 58.42) (width 1) (layer B.Cu) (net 14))
 (segment (start 212.0011 54.2036) (end 212.0011 58.3311) (width 1) (layer B.Cu) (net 14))
 (segment (start 209.4611 57.2389) (end 208.28 58.42) (width 1) (layer B.Cu) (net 15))
 (segment (start 209.4611 54.2036) (end 209.4611 57.2389) (width 1) (layer B.Cu) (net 15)))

